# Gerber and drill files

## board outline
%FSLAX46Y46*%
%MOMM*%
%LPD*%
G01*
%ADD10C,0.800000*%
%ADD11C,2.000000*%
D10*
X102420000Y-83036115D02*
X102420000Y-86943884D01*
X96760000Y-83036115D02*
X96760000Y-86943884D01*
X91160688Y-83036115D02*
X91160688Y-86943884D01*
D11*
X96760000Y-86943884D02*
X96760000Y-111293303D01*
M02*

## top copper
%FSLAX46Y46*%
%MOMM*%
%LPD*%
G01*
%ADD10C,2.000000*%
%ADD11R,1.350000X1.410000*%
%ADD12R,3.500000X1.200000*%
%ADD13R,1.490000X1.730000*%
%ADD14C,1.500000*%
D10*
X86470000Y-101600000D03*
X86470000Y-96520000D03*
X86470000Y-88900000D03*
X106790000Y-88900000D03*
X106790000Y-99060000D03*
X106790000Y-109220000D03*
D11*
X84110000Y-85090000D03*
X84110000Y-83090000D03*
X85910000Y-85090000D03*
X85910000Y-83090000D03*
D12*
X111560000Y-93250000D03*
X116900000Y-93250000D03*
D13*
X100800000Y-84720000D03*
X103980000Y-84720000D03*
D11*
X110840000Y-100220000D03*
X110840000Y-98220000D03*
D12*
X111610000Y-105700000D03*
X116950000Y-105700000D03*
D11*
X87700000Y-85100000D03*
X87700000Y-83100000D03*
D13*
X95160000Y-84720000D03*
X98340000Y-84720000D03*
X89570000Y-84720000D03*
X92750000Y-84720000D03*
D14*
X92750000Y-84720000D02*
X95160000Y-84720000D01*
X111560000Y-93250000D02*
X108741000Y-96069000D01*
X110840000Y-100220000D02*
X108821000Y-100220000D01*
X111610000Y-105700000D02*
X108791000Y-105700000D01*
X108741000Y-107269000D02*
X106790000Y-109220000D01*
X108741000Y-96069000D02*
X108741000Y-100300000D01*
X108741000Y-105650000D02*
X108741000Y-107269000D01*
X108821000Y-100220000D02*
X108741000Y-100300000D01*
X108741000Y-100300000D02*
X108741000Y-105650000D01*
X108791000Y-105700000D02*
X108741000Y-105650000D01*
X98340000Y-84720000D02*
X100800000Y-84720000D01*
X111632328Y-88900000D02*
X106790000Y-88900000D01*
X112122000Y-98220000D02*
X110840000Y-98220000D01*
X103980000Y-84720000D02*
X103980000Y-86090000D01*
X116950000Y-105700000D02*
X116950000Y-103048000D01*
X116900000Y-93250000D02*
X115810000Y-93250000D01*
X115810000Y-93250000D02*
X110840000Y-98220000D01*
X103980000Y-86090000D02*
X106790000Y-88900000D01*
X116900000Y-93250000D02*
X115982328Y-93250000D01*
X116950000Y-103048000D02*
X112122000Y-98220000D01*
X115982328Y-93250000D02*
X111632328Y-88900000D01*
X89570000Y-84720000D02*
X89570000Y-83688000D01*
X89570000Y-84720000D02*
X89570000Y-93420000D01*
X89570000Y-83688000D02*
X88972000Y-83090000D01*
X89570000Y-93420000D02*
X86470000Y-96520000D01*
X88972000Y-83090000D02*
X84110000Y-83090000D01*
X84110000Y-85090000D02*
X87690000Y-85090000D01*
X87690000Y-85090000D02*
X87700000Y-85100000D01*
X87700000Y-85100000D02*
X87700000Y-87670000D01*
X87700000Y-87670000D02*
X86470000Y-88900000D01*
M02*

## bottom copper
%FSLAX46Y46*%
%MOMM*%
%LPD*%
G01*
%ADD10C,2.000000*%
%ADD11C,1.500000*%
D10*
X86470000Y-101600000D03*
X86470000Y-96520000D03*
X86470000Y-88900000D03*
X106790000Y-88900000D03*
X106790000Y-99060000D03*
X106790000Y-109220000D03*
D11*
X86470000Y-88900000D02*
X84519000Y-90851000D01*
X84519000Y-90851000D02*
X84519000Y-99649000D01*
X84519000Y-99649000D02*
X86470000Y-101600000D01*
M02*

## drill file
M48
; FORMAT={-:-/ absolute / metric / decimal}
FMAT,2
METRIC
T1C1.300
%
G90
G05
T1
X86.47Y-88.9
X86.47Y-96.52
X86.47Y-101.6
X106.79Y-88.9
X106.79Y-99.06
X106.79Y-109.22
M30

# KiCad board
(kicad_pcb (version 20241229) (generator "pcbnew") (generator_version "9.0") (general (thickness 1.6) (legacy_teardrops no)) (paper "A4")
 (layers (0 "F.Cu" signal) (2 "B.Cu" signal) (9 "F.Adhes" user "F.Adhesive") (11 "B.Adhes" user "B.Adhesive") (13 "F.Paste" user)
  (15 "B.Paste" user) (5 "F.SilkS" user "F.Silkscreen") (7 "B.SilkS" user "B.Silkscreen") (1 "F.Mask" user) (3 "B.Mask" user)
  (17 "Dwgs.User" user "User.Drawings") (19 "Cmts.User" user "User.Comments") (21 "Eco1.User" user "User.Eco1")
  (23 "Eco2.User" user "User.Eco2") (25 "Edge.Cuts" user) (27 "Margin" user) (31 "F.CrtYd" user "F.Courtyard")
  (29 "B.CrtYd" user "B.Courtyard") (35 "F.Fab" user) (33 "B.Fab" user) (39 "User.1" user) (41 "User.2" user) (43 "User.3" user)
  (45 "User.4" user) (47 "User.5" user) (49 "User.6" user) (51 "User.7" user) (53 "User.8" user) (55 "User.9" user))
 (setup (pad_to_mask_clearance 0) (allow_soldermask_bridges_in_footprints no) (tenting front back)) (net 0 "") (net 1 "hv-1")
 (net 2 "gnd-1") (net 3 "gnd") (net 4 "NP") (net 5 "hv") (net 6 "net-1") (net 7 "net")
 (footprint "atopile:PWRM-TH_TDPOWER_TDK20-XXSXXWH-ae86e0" (layer "F.Cu") (at 96.63 99.06 0)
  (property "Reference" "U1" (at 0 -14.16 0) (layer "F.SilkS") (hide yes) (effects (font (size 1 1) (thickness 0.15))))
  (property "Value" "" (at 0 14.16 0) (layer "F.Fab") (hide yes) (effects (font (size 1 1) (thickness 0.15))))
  (pad "1" thru_hole circle (at -10.16 2.54 180) (size 2 2) (drill 1.300023) (layers "*.Cu" "*.Mask") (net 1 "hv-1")
   (remove_unused_layers no))
  (pad "2" thru_hole circle (at -10.16 -2.54 180) (size 2 2) (drill 1.300023) (layers "*.Cu" "*.Mask") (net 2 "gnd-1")
   (remove_unused_layers no))
  (pad "3" thru_hole circle (at -10.16 -10.16 180) (size 2 2) (drill 1.300023) (layers "*.Cu" "*.Mask") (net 1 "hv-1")
   (remove_unused_layers no))
  (pad "4" thru_hole circle (at 10.16 -10.16 180) (size 2 2) (drill 1.300023) (layers "*.Cu" "*.Mask") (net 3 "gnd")
   (remove_unused_layers no))
  (pad "5" thru_hole circle (at 10.16 0 180) (size 2 2) (drill 1.300023) (layers "*.Cu" "*.Mask") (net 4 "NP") (remove_unused_layers no))
  (pad "6" thru_hole circle (at 10.16 10.16 180) (size 2 2) (drill 1.300023) (layers "*.Cu" "*.Mask") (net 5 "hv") (remove_unused_layers no)))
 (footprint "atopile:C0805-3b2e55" (layer "F.Cu") (at 84.11 84.09 90)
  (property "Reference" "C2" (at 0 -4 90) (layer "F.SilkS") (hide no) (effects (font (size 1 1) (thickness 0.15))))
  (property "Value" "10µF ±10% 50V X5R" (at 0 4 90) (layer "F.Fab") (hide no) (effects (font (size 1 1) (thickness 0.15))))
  (pad "1" smd rect (at -1 0 90) (size 1.41 1.35) (layers "F.Cu" "F.Mask" "F.Paste") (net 1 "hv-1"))
  (pad "2" smd rect (at 1 0 90) (size 1.41 1.35) (layers "F.Cu" "F.Mask" "F.Paste") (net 2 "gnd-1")))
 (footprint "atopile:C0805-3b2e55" (layer "F.Cu") (at 85.91 84.09 90)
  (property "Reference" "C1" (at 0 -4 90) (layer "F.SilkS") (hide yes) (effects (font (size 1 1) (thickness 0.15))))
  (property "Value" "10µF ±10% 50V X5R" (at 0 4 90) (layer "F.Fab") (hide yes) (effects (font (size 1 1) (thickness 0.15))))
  (pad "1" smd rect (at -1 0 90) (size 1.41 1.35) (layers "F.Cu" "F.Mask" "F.Paste") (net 1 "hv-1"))
  (pad "2" smd rect (at 1 0 90) (size 1.41 1.35) (layers "F.Cu" "F.Mask" "F.Paste") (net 2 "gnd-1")))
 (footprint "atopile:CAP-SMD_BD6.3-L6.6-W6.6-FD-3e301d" (layer "F.Cu") (at 114.23 93.25 0)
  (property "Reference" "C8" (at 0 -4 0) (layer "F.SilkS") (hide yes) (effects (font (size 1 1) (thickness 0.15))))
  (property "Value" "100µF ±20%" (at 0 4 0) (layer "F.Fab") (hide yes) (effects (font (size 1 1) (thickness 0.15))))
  (pad "1" smd rect (at -2.67 0 0) (size 3.5 1.2) (layers "F.Cu" "F.Mask" "F.Paste") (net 5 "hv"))
  (pad "2" smd rect (at 2.67 0 0) (size 3.5 1.2) (layers "F.Cu" "F.Mask" "F.Paste") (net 3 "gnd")))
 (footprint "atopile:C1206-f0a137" (layer "F.Cu") (at 102.39 84.72 0)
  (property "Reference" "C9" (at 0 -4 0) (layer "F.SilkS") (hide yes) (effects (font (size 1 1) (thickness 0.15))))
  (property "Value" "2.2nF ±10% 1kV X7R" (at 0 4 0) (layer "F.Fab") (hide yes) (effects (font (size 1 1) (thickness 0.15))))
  (pad "1" smd rect (at -1.59 0 0) (size 1.49 1.73) (layers "F.Cu" "F.Mask" "F.Paste") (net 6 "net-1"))
  (pad "2" smd rect (at 1.59 0 0) (size 1.49 1.73) (layers "F.Cu" "F.Mask" "F.Paste") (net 3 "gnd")))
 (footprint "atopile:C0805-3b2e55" (layer "F.Cu") (at 110.84 99.22 90)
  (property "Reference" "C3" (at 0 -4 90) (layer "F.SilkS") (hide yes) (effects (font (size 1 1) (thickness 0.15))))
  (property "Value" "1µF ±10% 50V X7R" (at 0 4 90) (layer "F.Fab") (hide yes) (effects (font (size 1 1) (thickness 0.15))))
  (pad "1" smd rect (at -1 0 90) (size 1.41 1.35) (layers "F.Cu" "F.Mask" "F.Paste") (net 5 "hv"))
  (pad "2" smd rect (at 1 0 90) (size 1.41 1.35) (layers "F.Cu" "F.Mask" "F.Paste") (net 3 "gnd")))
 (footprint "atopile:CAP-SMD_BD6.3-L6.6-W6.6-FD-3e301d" (layer "F.Cu") (at 114.28 105.7 0)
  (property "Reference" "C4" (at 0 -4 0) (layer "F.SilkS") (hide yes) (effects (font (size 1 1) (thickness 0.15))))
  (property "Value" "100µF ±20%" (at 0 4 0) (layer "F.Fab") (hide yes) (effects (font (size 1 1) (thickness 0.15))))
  (pad "1" smd rect (at -2.67 0 0) (size 3.5 1.2) (layers "F.Cu" "F.Mask" "F.Paste") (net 5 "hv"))
  (pad "2" smd rect (at 2.67 0 0) (size 3.5 1.2) (layers "F.Cu" "F.Mask" "F.Paste") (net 3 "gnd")))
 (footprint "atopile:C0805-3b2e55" (layer "F.Cu") (at 87.7 84.1 90)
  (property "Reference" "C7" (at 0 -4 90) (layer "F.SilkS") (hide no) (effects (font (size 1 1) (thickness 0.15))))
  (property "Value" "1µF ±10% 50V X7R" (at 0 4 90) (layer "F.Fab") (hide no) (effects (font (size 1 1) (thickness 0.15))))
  (pad "1" smd rect (at -1 0 90) (size 1.41 1.35) (layers "F.Cu" "F.Mask" "F.Paste") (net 1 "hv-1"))
  (pad "2" smd rect (at 1 0 90) (size 1.41 1.35) (layers "F.Cu" "F.Mask" "F.Paste") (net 2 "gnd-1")))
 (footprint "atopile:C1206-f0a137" (layer "F.Cu") (at 96.75 84.72 0)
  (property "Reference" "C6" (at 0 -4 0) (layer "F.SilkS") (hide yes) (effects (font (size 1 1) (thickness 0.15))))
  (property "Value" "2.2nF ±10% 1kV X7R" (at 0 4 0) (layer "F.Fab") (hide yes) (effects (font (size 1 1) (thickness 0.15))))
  (pad "1" smd rect (at -1.59 0 0) (size 1.49 1.73) (layers "F.Cu" "F.Mask" "F.Paste") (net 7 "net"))
  (pad "2" smd rect (at 1.59 0 0) (size 1.49 1.73) (layers "F.Cu" "F.Mask" "F.Paste") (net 6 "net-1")))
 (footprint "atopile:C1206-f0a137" (layer "F.Cu") (at 91.16 84.72 0)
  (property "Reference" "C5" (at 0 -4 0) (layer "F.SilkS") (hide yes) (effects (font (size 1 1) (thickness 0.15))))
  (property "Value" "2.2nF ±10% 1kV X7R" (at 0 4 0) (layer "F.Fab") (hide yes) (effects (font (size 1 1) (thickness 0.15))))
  (pad "1" smd rect (at -1.59 0 0) (size 1.49 1.73) (layers "F.Cu" "F.Mask" "F.Paste") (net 2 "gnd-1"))
  (pad "2" smd rect (at 1.59 0 0) (size 1.49 1.73) (layers "F.Cu" "F.Mask" "F.Paste") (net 7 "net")))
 (segment (start 92.75 84.72) (end 95.16 84.72) (width 1.5) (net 7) (layer "F.Cu"))
 (segment (start 111.56 93.25) (end 108.741 96.069) (width 1.5) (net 5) (layer "F.Cu"))
 (segment (start 110.84 100.22) (end 108.821 100.22) (width 1.5) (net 5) (layer "F.Cu"))
 (segment (start 111.61 105.7) (end 108.791 105.7) (width 1.5) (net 5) (layer "F.Cu"))
 (segment (start 108.741 107.269) (end 106.79 109.22) (width 1.5) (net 5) (layer "F.Cu"))
 (segment (start 108.741 96.069) (end 108.741 100.3) (width 1.5) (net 5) (layer "F.Cu"))
 (segment (start 108.741 105.65) (end 108.741 107.269) (width 1.5) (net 5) (layer "F.Cu"))
 (segment (start 108.821 100.22) (end 108.741 100.3) (width 1.5) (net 5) (layer "F.Cu"))
 (segment (start 108.741 100.3) (end 108.741 105.65) (width 1.5) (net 5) (layer "F.Cu"))
 (segment (start 108.791 105.7) (end 108.741 105.65) (width 1.5) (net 5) (layer "F.Cu"))
 (segment (start 98.34 84.72) (end 100.8 84.72) (width 1.5) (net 6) (layer "F.Cu"))
 (segment (start 111.632328 88.9) (end 106.79 88.9) (width 1.5) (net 3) (layer "F.Cu"))
 (segment (start 112.122 98.22) (end 110.84 98.22) (width 1.5) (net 3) (layer "F.Cu"))
 (segment (start 103.98 84.72) (end 103.98 86.09) (width 1.5) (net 3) (layer "F.Cu"))
 (segment (start 116.95 105.7) (end 116.95 103.048) (width 1.5) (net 3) (layer "F.Cu"))
 (segment (start 116.9 93.25) (end 115.81 93.25) (width 1.5) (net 3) (layer "F.Cu"))
 (segment (start 115.81 93.25) (end 110.84 98.22) (width 1.5) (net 3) (layer "F.Cu"))
 (segment (start 103.98 86.09) (end 106.79 88.9) (width 1.5) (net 3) (layer "F.Cu"))
 (segment (start 116.9 93.25) (end 115.982328 93.25) (width 1.5) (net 3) (layer "F.Cu"))
 (segment (start 116.95 103.048) (end 112.122 98.22) (width 1.5) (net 3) (layer "F.Cu"))
 (segment (start 115.982328 93.25) (end 111.632328 88.9) (width 1.5) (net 3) (layer "F.Cu"))
 (segment (start 89.57 84.72) (end 89.57 83.688) (width 1.5) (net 2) (layer "F.Cu"))
 (segment (start 89.57 84.72) (end 89.57 93.42) (width 1.5) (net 2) (layer "F.Cu"))
 (segment (start 89.57 83.688) (end 88.972 83.09) (width 1.5) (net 2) (layer "F.Cu"))
 (segment (start 89.57 93.42) (end 86.47 96.52) (width 1.5) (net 2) (layer "F.Cu"))
 (segment (start 88.972 83.09) (end 84.11 83.09) (width 1.5) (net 2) (layer "F.Cu"))
 (segment (start 84.11 85.09) (end 87.69 85.09) (width 1.5) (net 1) (layer "F.Cu"))
 (segment (start 87.69 85.09) (end 87.7 85.1) (width 1.5) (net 1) (layer "F.Cu"))
 (segment (start 87.7 85.1) (end 87.7 87.67) (width 1.5) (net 1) (layer "F.Cu"))
 (segment (start 87.7 87.67) (end 86.47 88.9) (width 1.5) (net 1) (layer "F.Cu"))
 (segment (start 86.47 88.9) (end 84.519 90.851) (width 1.5) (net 1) (layer "B.Cu"))
 (segment (start 84.519 90.851) (end 84.519 99.649) (width 1.5) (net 1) (layer "B.Cu"))
 (segment (start 84.519 99.649) (end 86.47 101.6) (width 1.5) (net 1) (layer "B.Cu"))
 (gr_line (start 102.42 83.036115) (end 102.42 86.943884) (stroke (width 0.8) (type solid)) (layer "Edge.Cuts"))
 (gr_line (start 96.76 83.036115) (end 96.76 86.943884) (stroke (width 0.8) (type solid)) (layer "Edge.Cuts"))
 (gr_line (start 91.160688 83.036115) (end 91.160688 86.943884) (stroke (width 0.8) (type solid)) (layer "Edge.Cuts"))
 (gr_line (start 96.76 86.943884) (end 96.76 111.293303) (stroke (width 2) (type solid)) (layer "Edge.Cuts")))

